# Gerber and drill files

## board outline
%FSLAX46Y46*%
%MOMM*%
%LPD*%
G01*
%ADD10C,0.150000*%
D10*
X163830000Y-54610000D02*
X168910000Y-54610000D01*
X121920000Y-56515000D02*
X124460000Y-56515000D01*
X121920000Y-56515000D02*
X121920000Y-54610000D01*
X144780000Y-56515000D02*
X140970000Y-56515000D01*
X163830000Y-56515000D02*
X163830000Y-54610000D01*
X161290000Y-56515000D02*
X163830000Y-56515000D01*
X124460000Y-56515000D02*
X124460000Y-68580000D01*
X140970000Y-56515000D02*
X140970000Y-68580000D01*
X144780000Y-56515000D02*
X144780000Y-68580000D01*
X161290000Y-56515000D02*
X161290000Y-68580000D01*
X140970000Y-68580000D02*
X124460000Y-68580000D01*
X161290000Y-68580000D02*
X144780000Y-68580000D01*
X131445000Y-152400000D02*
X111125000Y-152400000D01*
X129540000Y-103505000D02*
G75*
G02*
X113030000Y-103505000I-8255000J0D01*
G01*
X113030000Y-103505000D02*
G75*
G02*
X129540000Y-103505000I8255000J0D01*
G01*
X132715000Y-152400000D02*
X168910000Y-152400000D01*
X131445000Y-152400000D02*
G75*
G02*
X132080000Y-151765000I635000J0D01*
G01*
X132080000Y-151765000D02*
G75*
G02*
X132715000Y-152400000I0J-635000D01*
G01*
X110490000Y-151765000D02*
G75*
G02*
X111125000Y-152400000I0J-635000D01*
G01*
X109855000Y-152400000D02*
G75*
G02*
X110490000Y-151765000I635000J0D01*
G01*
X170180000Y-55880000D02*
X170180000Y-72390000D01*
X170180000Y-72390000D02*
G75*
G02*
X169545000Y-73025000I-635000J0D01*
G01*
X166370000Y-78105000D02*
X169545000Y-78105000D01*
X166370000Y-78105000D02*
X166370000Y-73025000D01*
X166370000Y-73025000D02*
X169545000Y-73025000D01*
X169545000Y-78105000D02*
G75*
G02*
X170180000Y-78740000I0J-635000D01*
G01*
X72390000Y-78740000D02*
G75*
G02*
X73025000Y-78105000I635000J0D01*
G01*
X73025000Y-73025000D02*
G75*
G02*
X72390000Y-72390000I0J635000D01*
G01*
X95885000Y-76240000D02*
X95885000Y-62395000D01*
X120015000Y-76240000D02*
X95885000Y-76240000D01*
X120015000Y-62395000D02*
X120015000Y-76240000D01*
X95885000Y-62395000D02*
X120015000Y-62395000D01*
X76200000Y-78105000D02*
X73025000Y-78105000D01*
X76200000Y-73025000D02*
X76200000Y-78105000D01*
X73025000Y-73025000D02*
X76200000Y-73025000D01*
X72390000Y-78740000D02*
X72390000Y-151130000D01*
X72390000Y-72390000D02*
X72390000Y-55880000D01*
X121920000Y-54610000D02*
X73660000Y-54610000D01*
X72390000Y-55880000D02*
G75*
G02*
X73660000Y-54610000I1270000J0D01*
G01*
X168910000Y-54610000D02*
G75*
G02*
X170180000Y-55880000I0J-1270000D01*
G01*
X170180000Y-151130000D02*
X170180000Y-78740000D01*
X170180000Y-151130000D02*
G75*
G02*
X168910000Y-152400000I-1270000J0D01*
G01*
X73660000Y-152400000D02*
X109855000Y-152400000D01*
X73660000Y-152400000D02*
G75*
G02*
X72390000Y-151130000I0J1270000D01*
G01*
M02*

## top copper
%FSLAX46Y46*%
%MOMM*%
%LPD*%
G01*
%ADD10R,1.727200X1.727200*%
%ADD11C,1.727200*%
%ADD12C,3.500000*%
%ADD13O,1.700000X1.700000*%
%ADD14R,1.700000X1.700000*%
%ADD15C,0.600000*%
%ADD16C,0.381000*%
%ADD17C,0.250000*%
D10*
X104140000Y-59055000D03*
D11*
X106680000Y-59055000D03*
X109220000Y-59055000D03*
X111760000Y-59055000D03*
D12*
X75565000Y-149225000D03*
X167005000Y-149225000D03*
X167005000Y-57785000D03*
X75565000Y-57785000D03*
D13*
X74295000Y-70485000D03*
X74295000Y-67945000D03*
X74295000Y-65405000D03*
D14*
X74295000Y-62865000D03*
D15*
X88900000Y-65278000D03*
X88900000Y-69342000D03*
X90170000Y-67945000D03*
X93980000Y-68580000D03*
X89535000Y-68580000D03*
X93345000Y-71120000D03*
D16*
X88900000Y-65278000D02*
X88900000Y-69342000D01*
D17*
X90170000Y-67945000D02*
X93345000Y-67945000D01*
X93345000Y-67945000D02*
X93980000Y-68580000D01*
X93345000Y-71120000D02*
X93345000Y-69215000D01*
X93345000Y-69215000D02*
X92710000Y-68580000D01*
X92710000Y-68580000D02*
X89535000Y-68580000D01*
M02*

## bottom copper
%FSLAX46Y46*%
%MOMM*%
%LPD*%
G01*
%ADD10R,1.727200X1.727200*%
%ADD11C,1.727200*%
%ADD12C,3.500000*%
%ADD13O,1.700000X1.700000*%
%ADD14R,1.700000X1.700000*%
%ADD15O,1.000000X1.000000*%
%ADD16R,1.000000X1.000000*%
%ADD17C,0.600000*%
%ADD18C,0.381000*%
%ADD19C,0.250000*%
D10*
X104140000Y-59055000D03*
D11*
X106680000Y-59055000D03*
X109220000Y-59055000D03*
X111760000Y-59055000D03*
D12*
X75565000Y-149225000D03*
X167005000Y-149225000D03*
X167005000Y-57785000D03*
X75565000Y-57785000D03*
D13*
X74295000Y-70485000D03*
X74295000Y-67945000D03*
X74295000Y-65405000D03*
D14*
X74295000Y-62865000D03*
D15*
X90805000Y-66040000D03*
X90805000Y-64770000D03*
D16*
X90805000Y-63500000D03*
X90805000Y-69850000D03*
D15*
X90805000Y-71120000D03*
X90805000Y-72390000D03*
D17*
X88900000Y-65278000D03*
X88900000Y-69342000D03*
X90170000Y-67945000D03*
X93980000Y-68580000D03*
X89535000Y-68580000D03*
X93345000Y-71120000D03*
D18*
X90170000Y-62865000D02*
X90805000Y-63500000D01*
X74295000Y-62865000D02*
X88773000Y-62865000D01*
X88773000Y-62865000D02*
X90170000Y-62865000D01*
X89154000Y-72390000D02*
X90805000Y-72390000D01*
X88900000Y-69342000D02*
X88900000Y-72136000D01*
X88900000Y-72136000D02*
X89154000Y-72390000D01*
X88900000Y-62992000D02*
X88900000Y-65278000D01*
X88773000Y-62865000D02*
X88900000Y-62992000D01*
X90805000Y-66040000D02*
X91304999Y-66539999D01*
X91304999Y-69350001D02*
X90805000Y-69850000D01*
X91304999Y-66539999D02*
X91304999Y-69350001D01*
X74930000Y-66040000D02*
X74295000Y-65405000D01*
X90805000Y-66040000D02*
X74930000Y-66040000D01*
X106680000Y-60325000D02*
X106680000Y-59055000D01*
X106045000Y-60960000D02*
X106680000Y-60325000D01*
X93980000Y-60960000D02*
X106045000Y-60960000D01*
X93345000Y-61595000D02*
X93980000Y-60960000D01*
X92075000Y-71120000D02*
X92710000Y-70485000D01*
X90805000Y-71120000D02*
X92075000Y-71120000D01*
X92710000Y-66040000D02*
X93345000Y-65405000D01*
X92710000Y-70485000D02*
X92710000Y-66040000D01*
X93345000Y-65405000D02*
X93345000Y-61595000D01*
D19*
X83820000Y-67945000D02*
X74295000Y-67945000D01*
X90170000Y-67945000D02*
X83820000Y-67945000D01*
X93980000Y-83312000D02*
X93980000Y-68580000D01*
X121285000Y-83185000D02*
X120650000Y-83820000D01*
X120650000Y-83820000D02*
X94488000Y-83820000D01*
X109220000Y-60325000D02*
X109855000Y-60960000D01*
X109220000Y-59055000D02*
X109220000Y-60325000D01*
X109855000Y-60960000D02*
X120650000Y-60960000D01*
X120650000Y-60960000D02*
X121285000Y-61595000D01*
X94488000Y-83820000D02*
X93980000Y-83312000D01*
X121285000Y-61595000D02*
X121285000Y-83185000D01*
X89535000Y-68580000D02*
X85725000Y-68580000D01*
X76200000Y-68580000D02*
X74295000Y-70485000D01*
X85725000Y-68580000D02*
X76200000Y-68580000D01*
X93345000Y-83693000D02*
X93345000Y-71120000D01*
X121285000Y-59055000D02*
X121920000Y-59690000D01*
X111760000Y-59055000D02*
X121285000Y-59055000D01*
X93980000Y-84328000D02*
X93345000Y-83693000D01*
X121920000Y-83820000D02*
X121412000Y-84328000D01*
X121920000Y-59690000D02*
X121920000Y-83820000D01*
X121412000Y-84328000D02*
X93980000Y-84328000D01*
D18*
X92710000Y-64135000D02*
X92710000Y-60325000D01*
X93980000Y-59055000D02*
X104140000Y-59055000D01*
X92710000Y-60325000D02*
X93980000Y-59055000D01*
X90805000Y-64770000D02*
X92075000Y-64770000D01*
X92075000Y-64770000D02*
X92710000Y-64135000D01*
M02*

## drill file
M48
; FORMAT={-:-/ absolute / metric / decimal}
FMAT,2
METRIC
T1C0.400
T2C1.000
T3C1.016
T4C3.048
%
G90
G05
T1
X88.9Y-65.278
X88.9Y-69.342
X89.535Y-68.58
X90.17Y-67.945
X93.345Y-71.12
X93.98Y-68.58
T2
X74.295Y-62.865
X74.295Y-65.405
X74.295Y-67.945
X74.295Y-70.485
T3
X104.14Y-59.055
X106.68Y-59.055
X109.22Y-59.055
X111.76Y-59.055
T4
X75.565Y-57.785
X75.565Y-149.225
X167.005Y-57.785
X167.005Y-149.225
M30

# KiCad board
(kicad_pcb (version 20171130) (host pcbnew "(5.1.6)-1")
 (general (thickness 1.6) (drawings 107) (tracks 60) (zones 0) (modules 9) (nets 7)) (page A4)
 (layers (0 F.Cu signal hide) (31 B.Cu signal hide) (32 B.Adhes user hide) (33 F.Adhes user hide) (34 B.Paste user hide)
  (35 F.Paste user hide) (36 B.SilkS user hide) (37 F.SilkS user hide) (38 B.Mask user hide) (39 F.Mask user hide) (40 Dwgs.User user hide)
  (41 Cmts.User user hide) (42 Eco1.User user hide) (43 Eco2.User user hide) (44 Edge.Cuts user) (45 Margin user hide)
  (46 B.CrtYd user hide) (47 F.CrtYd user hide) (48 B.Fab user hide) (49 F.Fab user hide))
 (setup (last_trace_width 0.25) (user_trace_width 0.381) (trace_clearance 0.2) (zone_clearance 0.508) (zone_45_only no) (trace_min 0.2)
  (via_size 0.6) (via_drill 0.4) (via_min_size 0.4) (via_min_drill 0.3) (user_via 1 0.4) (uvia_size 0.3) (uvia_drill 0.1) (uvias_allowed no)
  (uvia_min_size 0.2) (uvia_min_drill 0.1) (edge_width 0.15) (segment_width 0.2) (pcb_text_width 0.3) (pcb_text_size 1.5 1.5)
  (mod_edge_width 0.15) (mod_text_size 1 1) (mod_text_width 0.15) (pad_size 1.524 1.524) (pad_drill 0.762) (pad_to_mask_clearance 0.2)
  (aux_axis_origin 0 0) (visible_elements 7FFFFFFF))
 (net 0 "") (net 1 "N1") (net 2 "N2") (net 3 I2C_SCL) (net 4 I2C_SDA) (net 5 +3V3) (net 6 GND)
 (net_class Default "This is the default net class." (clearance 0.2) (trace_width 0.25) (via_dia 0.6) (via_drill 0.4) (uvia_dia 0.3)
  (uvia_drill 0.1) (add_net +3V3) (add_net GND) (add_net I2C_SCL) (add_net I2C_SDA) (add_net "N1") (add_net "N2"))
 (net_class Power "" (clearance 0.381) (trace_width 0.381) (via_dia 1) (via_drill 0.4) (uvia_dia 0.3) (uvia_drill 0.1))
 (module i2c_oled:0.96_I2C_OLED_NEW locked (layer F.Cu) (at 107.95 59.055)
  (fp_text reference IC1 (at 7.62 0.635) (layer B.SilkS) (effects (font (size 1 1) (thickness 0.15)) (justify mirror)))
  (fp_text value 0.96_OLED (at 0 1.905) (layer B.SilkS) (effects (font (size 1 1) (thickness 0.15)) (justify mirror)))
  (pad 1 thru_hole rect (at -3.81 0) (size 1.7272 1.7272) (drill 1.016) (layers *.Cu *.Mask) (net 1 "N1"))
  (pad 2 thru_hole circle (at -1.27 0) (size 1.7272 1.7272) (drill 1.016) (layers *.Cu *.Mask) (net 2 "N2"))
  (pad 3 thru_hole circle (at 1.27 0) (size 1.7272 1.7272) (drill 1.016) (layers *.Cu *.Mask) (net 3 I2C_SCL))
  (pad 4 thru_hole circle (at 3.81 0) (size 1.7272 1.7272) (drill 1.016) (layers *.Cu *.Mask) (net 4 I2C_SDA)))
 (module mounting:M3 (layer F.Cu) (at 75.565 149.225)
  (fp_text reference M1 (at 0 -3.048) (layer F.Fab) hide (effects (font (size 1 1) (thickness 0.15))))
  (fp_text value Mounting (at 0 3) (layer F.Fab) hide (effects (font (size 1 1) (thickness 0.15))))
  (pad "" np_thru_hole circle (at 0 0) (size 3.5 3.5) (drill 3.048) (layers *.Cu *.Mask) (solder_mask_margin 0.8)))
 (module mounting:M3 (layer F.Cu) (at 167.005 149.225)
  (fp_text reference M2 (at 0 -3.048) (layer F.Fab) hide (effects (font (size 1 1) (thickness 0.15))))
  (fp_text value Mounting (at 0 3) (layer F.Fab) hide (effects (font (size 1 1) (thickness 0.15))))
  (pad "" np_thru_hole circle (at 0 0) (size 3.5 3.5) (drill 3.048) (layers *.Cu *.Mask) (solder_mask_margin 0.8)))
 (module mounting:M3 (layer F.Cu) (at 167.005 57.785)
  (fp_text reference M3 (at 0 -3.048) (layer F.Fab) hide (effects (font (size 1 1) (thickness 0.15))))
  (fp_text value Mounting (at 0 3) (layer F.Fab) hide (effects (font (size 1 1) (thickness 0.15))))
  (pad "" np_thru_hole circle (at 0 0) (size 3.5 3.5) (drill 3.048) (layers *.Cu *.Mask) (solder_mask_margin 0.8)))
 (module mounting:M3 (layer F.Cu) (at 75.565 57.785)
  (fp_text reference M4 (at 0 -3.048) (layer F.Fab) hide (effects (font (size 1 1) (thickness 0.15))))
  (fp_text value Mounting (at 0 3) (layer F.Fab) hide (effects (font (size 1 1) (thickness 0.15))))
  (pad "" np_thru_hole circle (at 0 0) (size 3.5 3.5) (drill 3.048) (layers *.Cu *.Mask) (solder_mask_margin 0.8)))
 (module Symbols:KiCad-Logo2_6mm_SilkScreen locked (layer B.Cu) (at 153.205 92.95 180)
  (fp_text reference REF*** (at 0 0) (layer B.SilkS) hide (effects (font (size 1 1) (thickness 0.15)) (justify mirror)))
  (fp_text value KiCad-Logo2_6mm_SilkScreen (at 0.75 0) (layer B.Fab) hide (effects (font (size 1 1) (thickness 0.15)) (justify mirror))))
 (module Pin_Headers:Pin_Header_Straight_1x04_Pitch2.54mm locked (layer B.Cu) (at 74.295 62.865 180)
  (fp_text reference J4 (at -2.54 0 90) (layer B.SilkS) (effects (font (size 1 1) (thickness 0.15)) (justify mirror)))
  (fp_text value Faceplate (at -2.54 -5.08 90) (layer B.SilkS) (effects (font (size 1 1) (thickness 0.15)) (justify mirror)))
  (pad 4 thru_hole oval (at 0 -7.62 180) (size 1.7 1.7) (drill 1) (layers *.Cu *.Mask) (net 4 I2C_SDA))
  (pad 3 thru_hole oval (at 0 -5.08 180) (size 1.7 1.7) (drill 1) (layers *.Cu *.Mask) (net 3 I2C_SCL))
  (pad 2 thru_hole oval (at 0 -2.54 180) (size 1.7 1.7) (drill 1) (layers *.Cu *.Mask) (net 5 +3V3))
  (pad 1 thru_hole rect (at 0 0 180) (size 1.7 1.7) (drill 1) (layers *.Cu *.Mask) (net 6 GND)))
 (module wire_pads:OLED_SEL (layer B.Cu) (at 90.805 63.5 180)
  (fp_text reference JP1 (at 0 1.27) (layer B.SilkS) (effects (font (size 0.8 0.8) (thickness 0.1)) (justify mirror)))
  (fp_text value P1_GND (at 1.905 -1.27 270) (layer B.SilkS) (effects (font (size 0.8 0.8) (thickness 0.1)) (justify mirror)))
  (pad 3 smd oval (at 0 -2.54 180) (size 1 1) (layers B.Cu B.Paste B.Mask) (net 5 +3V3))
  (pad 2 smd oval (at 0 -1.27 180) (size 1 1) (layers B.Cu B.Paste B.Mask) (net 1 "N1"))
  (pad 1 smd rect (at 0 0 180) (size 1 1) (layers B.Cu B.Paste B.Mask) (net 6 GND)))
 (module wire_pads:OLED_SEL (layer B.Cu) (at 90.805 69.85 180)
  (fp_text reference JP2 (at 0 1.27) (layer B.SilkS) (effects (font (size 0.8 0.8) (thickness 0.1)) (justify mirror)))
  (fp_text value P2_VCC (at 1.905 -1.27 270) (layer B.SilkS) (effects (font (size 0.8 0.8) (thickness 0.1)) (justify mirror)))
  (pad 1 smd rect (at 0 0 180) (size 1 1) (layers B.Cu B.Paste B.Mask) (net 5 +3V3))
  (pad 2 smd oval (at 0 -1.27 180) (size 1 1) (layers B.Cu B.Paste B.Mask) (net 2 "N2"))
  (pad 3 smd oval (at 0 -2.54 180) (size 1 1) (layers B.Cu B.Paste B.Mask) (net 6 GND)))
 (gr_line (start 163.83 54.61) (end 168.91 54.61) (layer Edge.Cuts) (width 0.15))
 (gr_line (start 121.92 56.515) (end 124.46 56.515) (layer Edge.Cuts) (width 0.15))
 (gr_line (start 121.92 56.515) (end 121.92 54.61) (layer Edge.Cuts) (width 0.15))
 (gr_line (start 144.78 56.515) (end 140.97 56.515) (layer Edge.Cuts) (width 0.15))
 (gr_line (start 163.83 56.515) (end 163.83 54.61) (layer Edge.Cuts) (width 0.15))
 (gr_line (start 161.29 56.515) (end 163.83 56.515) (layer Edge.Cuts) (width 0.15))
 (gr_line (start 124.46 56.515) (end 124.46 68.58) (layer Edge.Cuts) (width 0.15))
 (gr_line (start 140.97 56.515) (end 140.97 68.58) (layer Edge.Cuts) (width 0.15))
 (gr_line (start 144.78 56.515) (end 144.78 68.58) (layer Edge.Cuts) (width 0.15))
 (gr_line (start 161.29 56.515) (end 161.29 68.58) (layer Edge.Cuts) (width 0.15))
 (gr_line (start 140.97 68.58) (end 124.46 68.58) (layer Edge.Cuts) (width 0.15))
 (gr_line (start 161.29 68.58) (end 144.78 68.58) (layer Edge.Cuts) (width 0.15))
 (gr_line (start 131.445 152.4) (end 111.125 152.4) (layer Edge.Cuts) (width 0.15))
 (gr_circle (center 121.285 103.505) (end 129.54 103.505) (layer Edge.Cuts) (width 0.15))
 (gr_line (start 132.715 152.4) (end 168.91 152.4) (layer Edge.Cuts) (width 0.15))
 (gr_arc (start 132.08 152.4) (end 132.08 151.765) (angle -90) (layer Edge.Cuts) (width 0.15))
 (gr_arc (start 132.08 152.4) (end 132.715 152.4) (angle -90) (layer Edge.Cuts) (width 0.15))
 (gr_arc (start 110.49 152.4) (end 111.125 152.4) (angle -90) (layer Edge.Cuts) (width 0.15))
 (gr_arc (start 110.49 152.4) (end 110.49 151.765) (angle -90) (layer Edge.Cuts) (width 0.15))
 (gr_line (start 170.18 55.88) (end 170.18 72.39) (layer Edge.Cuts) (width 0.15))
 (gr_arc (start 169.545 72.39) (end 169.545 73.025) (angle -90) (layer Edge.Cuts) (width 0.15))
 (gr_line (start 166.37 78.105) (end 169.545 78.105) (layer Edge.Cuts) (width 0.15))
 (gr_line (start 166.37 78.105) (end 166.37 73.025) (layer Edge.Cuts) (width 0.15))
 (gr_line (start 166.37 73.025) (end 169.545 73.025) (layer Edge.Cuts) (width 0.15))
 (gr_arc (start 169.545 78.74) (end 170.18 78.74) (angle -90) (layer Edge.Cuts) (width 0.15))
 (gr_arc (start 73.025 78.74) (end 73.025 78.105) (angle -90) (layer Edge.Cuts) (width 0.15))
 (gr_arc (start 73.025 72.39) (end 72.39 72.39) (angle -90) (layer Edge.Cuts) (width 0.15))
 (gr_line (start 95.885 76.24) (end 95.885 62.395) (layer Edge.Cuts) (width 0.15))
 (gr_line (start 120.015 76.24) (end 95.885 76.24) (layer Edge.Cuts) (width 0.15))
 (gr_line (start 120.015 62.395) (end 120.015 76.24) (layer Edge.Cuts) (width 0.15))
 (gr_line (start 95.885 62.395) (end 120.015 62.395) (layer Edge.Cuts) (width 0.15))
 (gr_line (start 76.2 78.105) (end 73.025 78.105) (layer Edge.Cuts) (width 0.15))
 (gr_line (start 76.2 73.025) (end 76.2 78.105) (layer Edge.Cuts) (width 0.15))
 (gr_line (start 73.025 73.025) (end 76.2 73.025) (layer Edge.Cuts) (width 0.15))
 (gr_line (start 72.39 78.74) (end 72.39 151.13) (layer Edge.Cuts) (width 0.15))
 (gr_line (start 72.39 72.39) (end 72.39 55.88) (layer Edge.Cuts) (width 0.15))
 (gr_line (start 121.92 54.61) (end 73.66 54.61) (angle 90) (layer Edge.Cuts) (width 0.15))
 (gr_arc (start 73.66 55.88) (end 72.39 55.88) (angle 90) (layer Edge.Cuts) (width 0.15))
 (gr_arc (start 168.91 55.88) (end 168.91 54.61) (angle 90) (layer Edge.Cuts) (width 0.15))
 (gr_line (start 170.18 151.13) (end 170.18 78.74) (angle 90) (layer Edge.Cuts) (width 0.15))
 (gr_arc (start 168.91 151.13) (end 170.18 151.13) (angle 90) (layer Edge.Cuts) (width 0.15))
 (gr_line (start 73.66 152.4) (end 109.855 152.4) (angle 90) (layer Edge.Cuts) (width 0.15))
 (gr_arc (start 73.66 151.13) (end 73.66 152.4) (angle 90) (layer Edge.Cuts) (width 0.15))
 (segment (start 90.17 62.865) (end 90.805 63.5) (width 0.381) (layer B.Cu) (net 6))
 (via (at 88.9 65.278) (size 0.6) (drill 0.4) (layers F.Cu B.Cu) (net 6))
 (segment (start 74.295 62.865) (end 88.773 62.865) (width 0.381) (layer B.Cu) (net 6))
 (segment (start 88.773 62.865) (end 90.17 62.865) (width 0.381) (layer B.Cu) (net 6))
 (via (at 88.9 69.342) (size 0.6) (drill 0.4) (layers F.Cu B.Cu) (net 6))
 (segment (start 88.9 65.278) (end 88.9 69.342) (width 0.381) (layer F.Cu) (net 6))
 (segment (start 89.154 72.39) (end 90.805 72.39) (width 0.381) (layer B.Cu) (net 6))
 (segment (start 88.9 69.342) (end 88.9 72.136) (width 0.381) (layer B.Cu) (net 6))
 (segment (start 88.9 72.136) (end 89.154 72.39) (width 0.381) (layer B.Cu) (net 6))
 (segment (start 88.9 62.992) (end 88.9 65.278) (width 0.381) (layer B.Cu) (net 6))
 (segment (start 88.773 62.865) (end 88.9 62.992) (width 0.381) (layer B.Cu) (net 6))
 (segment (start 90.805 66.04) (end 91.304999 66.539999) (width 0.381) (layer B.Cu) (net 5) (status 10))
 (segment (start 91.304999 69.350001) (end 90.805 69.85) (width 0.381) (layer B.Cu) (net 5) (status 30))
 (segment (start 91.304999 66.539999) (end 91.304999 69.350001) (width 0.381) (layer B.Cu) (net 5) (status 20))
 (segment (start 74.93 66.04) (end 74.295 65.405) (width 0.381) (layer B.Cu) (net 5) (status 20))
 (segment (start 90.805 66.04) (end 74.93 66.04) (width 0.381) (layer B.Cu) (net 5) (status 10))
 (segment (start 106.68 60.325) (end 106.68 59.055) (width 0.381) (layer B.Cu) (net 2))
 (segment (start 106.045 60.96) (end 106.68 60.325) (width 0.381) (layer B.Cu) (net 2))
 (segment (start 93.98 60.96) (end 106.045 60.96) (width 0.381) (layer B.Cu) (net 2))
 (segment (start 93.345 61.595) (end 93.98 60.96) (width 0.381) (layer B.Cu) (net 2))
 (segment (start 92.075 71.12) (end 92.71 70.485) (width 0.381) (layer B.Cu) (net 2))
 (segment (start 90.805 71.12) (end 92.075 71.12) (width 0.381) (layer B.Cu) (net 2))
 (segment (start 92.71 66.04) (end 93.345 65.405) (width 0.381) (layer B.Cu) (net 2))
 (segment (start 92.71 70.485) (end 92.71 66.04) (width 0.381) (layer B.Cu) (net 2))
 (segment (start 93.345 65.405) (end 93.345 61.595) (width 0.381) (layer B.Cu) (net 2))
 (via (at 90.17 67.945) (size 0.6) (drill 0.4) (layers F.Cu B.Cu) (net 3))
 (segment (start 90.17 67.945) (end 93.345 67.945) (width 0.25) (layer F.Cu) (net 3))
 (segment (start 83.82 67.945) (end 74.295 67.945) (width 0.25) (layer B.Cu) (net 3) (status 20))
 (segment (start 90.17 67.945) (end 83.82 67.945) (width 0.25) (layer B.Cu) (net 3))
 (via (at 93.98 68.58) (size 0.6) (drill 0.4) (layers F.Cu B.Cu) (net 3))
 (segment (start 93.345 67.945) (end 93.98 68.58) (width 0.25) (layer F.Cu) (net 3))
 (segment (start 93.98 83.312) (end 93.98 68.58) (width 0.25) (layer B.Cu) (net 3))
 (segment (start 121.285 83.185) (end 120.65 83.82) (width 0.25) (layer B.Cu) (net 3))
 (segment (start 120.65 83.82) (end 94.488 83.82) (width 0.25) (layer B.Cu) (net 3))
 (segment (start 109.22 60.325) (end 109.855 60.96) (width 0.25) (layer B.Cu) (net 3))
 (segment (start 109.22 59.055) (end 109.22 60.325) (width 0.25) (layer B.Cu) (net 3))
 (segment (start 109.855 60.96) (end 120.65 60.96) (width 0.25) (layer B.Cu) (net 3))
 (segment (start 120.65 60.96) (end 121.285 61.595) (width 0.25) (layer B.Cu) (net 3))
 (segment (start 94.488 83.82) (end 93.98 83.312) (width 0.25) (layer B.Cu) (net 3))
 (segment (start 121.285 61.595) (end 121.285 83.185) (width 0.25) (layer B.Cu) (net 3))
 (via (at 89.535 68.58) (size 0.6) (drill 0.4) (layers F.Cu B.Cu) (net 4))
 (segment (start 89.535 68.58) (end 85.725 68.58) (width 0.25) (layer B.Cu) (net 4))
 (segment (start 76.2 68.58) (end 74.295 70.485) (width 0.25) (layer B.Cu) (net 4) (status 20))
 (segment (start 85.725 68.58) (end 76.2 68.58) (width 0.25) (layer B.Cu) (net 4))
 (via (at 93.345 71.12) (size 0.6) (drill 0.4) (layers F.Cu B.Cu) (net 4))
 (segment (start 93.345 71.12) (end 93.345 69.215) (width 0.25) (layer F.Cu) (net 4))
 (segment (start 93.345 69.215) (end 92.71 68.58) (width 0.25) (layer F.Cu) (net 4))
 (segment (start 92.71 68.58) (end 89.535 68.58) (width 0.25) (layer F.Cu) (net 4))
 (segment (start 93.345 83.693) (end 93.345 71.12) (width 0.25) (layer B.Cu) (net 4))
 (segment (start 121.285 59.055) (end 121.92 59.69) (width 0.25) (layer B.Cu) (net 4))
 (segment (start 111.76 59.055) (end 121.285 59.055) (width 0.25) (layer B.Cu) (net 4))
 (segment (start 93.98 84.328) (end 93.345 83.693) (width 0.25) (layer B.Cu) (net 4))
 (segment (start 121.92 83.82) (end 121.412 84.328) (width 0.25) (layer B.Cu) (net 4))
 (segment (start 121.92 59.69) (end 121.92 83.82) (width 0.25) (layer B.Cu) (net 4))
 (segment (start 121.412 84.328) (end 93.98 84.328) (width 0.25) (layer B.Cu) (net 4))
 (segment (start 92.71 64.135) (end 92.71 60.325) (width 0.381) (layer B.Cu) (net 1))
 (segment (start 93.98 59.055) (end 104.14 59.055) (width 0.381) (layer B.Cu) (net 1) (status 20))
 (segment (start 92.71 60.325) (end 93.98 59.055) (width 0.381) (layer B.Cu) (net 1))
 (segment (start 90.805 64.77) (end 92.075 64.77) (width 0.381) (layer B.Cu) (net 1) (status 10))
 (segment (start 92.075 64.77) (end 92.71 64.135) (width 0.381) (layer B.Cu) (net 1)))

